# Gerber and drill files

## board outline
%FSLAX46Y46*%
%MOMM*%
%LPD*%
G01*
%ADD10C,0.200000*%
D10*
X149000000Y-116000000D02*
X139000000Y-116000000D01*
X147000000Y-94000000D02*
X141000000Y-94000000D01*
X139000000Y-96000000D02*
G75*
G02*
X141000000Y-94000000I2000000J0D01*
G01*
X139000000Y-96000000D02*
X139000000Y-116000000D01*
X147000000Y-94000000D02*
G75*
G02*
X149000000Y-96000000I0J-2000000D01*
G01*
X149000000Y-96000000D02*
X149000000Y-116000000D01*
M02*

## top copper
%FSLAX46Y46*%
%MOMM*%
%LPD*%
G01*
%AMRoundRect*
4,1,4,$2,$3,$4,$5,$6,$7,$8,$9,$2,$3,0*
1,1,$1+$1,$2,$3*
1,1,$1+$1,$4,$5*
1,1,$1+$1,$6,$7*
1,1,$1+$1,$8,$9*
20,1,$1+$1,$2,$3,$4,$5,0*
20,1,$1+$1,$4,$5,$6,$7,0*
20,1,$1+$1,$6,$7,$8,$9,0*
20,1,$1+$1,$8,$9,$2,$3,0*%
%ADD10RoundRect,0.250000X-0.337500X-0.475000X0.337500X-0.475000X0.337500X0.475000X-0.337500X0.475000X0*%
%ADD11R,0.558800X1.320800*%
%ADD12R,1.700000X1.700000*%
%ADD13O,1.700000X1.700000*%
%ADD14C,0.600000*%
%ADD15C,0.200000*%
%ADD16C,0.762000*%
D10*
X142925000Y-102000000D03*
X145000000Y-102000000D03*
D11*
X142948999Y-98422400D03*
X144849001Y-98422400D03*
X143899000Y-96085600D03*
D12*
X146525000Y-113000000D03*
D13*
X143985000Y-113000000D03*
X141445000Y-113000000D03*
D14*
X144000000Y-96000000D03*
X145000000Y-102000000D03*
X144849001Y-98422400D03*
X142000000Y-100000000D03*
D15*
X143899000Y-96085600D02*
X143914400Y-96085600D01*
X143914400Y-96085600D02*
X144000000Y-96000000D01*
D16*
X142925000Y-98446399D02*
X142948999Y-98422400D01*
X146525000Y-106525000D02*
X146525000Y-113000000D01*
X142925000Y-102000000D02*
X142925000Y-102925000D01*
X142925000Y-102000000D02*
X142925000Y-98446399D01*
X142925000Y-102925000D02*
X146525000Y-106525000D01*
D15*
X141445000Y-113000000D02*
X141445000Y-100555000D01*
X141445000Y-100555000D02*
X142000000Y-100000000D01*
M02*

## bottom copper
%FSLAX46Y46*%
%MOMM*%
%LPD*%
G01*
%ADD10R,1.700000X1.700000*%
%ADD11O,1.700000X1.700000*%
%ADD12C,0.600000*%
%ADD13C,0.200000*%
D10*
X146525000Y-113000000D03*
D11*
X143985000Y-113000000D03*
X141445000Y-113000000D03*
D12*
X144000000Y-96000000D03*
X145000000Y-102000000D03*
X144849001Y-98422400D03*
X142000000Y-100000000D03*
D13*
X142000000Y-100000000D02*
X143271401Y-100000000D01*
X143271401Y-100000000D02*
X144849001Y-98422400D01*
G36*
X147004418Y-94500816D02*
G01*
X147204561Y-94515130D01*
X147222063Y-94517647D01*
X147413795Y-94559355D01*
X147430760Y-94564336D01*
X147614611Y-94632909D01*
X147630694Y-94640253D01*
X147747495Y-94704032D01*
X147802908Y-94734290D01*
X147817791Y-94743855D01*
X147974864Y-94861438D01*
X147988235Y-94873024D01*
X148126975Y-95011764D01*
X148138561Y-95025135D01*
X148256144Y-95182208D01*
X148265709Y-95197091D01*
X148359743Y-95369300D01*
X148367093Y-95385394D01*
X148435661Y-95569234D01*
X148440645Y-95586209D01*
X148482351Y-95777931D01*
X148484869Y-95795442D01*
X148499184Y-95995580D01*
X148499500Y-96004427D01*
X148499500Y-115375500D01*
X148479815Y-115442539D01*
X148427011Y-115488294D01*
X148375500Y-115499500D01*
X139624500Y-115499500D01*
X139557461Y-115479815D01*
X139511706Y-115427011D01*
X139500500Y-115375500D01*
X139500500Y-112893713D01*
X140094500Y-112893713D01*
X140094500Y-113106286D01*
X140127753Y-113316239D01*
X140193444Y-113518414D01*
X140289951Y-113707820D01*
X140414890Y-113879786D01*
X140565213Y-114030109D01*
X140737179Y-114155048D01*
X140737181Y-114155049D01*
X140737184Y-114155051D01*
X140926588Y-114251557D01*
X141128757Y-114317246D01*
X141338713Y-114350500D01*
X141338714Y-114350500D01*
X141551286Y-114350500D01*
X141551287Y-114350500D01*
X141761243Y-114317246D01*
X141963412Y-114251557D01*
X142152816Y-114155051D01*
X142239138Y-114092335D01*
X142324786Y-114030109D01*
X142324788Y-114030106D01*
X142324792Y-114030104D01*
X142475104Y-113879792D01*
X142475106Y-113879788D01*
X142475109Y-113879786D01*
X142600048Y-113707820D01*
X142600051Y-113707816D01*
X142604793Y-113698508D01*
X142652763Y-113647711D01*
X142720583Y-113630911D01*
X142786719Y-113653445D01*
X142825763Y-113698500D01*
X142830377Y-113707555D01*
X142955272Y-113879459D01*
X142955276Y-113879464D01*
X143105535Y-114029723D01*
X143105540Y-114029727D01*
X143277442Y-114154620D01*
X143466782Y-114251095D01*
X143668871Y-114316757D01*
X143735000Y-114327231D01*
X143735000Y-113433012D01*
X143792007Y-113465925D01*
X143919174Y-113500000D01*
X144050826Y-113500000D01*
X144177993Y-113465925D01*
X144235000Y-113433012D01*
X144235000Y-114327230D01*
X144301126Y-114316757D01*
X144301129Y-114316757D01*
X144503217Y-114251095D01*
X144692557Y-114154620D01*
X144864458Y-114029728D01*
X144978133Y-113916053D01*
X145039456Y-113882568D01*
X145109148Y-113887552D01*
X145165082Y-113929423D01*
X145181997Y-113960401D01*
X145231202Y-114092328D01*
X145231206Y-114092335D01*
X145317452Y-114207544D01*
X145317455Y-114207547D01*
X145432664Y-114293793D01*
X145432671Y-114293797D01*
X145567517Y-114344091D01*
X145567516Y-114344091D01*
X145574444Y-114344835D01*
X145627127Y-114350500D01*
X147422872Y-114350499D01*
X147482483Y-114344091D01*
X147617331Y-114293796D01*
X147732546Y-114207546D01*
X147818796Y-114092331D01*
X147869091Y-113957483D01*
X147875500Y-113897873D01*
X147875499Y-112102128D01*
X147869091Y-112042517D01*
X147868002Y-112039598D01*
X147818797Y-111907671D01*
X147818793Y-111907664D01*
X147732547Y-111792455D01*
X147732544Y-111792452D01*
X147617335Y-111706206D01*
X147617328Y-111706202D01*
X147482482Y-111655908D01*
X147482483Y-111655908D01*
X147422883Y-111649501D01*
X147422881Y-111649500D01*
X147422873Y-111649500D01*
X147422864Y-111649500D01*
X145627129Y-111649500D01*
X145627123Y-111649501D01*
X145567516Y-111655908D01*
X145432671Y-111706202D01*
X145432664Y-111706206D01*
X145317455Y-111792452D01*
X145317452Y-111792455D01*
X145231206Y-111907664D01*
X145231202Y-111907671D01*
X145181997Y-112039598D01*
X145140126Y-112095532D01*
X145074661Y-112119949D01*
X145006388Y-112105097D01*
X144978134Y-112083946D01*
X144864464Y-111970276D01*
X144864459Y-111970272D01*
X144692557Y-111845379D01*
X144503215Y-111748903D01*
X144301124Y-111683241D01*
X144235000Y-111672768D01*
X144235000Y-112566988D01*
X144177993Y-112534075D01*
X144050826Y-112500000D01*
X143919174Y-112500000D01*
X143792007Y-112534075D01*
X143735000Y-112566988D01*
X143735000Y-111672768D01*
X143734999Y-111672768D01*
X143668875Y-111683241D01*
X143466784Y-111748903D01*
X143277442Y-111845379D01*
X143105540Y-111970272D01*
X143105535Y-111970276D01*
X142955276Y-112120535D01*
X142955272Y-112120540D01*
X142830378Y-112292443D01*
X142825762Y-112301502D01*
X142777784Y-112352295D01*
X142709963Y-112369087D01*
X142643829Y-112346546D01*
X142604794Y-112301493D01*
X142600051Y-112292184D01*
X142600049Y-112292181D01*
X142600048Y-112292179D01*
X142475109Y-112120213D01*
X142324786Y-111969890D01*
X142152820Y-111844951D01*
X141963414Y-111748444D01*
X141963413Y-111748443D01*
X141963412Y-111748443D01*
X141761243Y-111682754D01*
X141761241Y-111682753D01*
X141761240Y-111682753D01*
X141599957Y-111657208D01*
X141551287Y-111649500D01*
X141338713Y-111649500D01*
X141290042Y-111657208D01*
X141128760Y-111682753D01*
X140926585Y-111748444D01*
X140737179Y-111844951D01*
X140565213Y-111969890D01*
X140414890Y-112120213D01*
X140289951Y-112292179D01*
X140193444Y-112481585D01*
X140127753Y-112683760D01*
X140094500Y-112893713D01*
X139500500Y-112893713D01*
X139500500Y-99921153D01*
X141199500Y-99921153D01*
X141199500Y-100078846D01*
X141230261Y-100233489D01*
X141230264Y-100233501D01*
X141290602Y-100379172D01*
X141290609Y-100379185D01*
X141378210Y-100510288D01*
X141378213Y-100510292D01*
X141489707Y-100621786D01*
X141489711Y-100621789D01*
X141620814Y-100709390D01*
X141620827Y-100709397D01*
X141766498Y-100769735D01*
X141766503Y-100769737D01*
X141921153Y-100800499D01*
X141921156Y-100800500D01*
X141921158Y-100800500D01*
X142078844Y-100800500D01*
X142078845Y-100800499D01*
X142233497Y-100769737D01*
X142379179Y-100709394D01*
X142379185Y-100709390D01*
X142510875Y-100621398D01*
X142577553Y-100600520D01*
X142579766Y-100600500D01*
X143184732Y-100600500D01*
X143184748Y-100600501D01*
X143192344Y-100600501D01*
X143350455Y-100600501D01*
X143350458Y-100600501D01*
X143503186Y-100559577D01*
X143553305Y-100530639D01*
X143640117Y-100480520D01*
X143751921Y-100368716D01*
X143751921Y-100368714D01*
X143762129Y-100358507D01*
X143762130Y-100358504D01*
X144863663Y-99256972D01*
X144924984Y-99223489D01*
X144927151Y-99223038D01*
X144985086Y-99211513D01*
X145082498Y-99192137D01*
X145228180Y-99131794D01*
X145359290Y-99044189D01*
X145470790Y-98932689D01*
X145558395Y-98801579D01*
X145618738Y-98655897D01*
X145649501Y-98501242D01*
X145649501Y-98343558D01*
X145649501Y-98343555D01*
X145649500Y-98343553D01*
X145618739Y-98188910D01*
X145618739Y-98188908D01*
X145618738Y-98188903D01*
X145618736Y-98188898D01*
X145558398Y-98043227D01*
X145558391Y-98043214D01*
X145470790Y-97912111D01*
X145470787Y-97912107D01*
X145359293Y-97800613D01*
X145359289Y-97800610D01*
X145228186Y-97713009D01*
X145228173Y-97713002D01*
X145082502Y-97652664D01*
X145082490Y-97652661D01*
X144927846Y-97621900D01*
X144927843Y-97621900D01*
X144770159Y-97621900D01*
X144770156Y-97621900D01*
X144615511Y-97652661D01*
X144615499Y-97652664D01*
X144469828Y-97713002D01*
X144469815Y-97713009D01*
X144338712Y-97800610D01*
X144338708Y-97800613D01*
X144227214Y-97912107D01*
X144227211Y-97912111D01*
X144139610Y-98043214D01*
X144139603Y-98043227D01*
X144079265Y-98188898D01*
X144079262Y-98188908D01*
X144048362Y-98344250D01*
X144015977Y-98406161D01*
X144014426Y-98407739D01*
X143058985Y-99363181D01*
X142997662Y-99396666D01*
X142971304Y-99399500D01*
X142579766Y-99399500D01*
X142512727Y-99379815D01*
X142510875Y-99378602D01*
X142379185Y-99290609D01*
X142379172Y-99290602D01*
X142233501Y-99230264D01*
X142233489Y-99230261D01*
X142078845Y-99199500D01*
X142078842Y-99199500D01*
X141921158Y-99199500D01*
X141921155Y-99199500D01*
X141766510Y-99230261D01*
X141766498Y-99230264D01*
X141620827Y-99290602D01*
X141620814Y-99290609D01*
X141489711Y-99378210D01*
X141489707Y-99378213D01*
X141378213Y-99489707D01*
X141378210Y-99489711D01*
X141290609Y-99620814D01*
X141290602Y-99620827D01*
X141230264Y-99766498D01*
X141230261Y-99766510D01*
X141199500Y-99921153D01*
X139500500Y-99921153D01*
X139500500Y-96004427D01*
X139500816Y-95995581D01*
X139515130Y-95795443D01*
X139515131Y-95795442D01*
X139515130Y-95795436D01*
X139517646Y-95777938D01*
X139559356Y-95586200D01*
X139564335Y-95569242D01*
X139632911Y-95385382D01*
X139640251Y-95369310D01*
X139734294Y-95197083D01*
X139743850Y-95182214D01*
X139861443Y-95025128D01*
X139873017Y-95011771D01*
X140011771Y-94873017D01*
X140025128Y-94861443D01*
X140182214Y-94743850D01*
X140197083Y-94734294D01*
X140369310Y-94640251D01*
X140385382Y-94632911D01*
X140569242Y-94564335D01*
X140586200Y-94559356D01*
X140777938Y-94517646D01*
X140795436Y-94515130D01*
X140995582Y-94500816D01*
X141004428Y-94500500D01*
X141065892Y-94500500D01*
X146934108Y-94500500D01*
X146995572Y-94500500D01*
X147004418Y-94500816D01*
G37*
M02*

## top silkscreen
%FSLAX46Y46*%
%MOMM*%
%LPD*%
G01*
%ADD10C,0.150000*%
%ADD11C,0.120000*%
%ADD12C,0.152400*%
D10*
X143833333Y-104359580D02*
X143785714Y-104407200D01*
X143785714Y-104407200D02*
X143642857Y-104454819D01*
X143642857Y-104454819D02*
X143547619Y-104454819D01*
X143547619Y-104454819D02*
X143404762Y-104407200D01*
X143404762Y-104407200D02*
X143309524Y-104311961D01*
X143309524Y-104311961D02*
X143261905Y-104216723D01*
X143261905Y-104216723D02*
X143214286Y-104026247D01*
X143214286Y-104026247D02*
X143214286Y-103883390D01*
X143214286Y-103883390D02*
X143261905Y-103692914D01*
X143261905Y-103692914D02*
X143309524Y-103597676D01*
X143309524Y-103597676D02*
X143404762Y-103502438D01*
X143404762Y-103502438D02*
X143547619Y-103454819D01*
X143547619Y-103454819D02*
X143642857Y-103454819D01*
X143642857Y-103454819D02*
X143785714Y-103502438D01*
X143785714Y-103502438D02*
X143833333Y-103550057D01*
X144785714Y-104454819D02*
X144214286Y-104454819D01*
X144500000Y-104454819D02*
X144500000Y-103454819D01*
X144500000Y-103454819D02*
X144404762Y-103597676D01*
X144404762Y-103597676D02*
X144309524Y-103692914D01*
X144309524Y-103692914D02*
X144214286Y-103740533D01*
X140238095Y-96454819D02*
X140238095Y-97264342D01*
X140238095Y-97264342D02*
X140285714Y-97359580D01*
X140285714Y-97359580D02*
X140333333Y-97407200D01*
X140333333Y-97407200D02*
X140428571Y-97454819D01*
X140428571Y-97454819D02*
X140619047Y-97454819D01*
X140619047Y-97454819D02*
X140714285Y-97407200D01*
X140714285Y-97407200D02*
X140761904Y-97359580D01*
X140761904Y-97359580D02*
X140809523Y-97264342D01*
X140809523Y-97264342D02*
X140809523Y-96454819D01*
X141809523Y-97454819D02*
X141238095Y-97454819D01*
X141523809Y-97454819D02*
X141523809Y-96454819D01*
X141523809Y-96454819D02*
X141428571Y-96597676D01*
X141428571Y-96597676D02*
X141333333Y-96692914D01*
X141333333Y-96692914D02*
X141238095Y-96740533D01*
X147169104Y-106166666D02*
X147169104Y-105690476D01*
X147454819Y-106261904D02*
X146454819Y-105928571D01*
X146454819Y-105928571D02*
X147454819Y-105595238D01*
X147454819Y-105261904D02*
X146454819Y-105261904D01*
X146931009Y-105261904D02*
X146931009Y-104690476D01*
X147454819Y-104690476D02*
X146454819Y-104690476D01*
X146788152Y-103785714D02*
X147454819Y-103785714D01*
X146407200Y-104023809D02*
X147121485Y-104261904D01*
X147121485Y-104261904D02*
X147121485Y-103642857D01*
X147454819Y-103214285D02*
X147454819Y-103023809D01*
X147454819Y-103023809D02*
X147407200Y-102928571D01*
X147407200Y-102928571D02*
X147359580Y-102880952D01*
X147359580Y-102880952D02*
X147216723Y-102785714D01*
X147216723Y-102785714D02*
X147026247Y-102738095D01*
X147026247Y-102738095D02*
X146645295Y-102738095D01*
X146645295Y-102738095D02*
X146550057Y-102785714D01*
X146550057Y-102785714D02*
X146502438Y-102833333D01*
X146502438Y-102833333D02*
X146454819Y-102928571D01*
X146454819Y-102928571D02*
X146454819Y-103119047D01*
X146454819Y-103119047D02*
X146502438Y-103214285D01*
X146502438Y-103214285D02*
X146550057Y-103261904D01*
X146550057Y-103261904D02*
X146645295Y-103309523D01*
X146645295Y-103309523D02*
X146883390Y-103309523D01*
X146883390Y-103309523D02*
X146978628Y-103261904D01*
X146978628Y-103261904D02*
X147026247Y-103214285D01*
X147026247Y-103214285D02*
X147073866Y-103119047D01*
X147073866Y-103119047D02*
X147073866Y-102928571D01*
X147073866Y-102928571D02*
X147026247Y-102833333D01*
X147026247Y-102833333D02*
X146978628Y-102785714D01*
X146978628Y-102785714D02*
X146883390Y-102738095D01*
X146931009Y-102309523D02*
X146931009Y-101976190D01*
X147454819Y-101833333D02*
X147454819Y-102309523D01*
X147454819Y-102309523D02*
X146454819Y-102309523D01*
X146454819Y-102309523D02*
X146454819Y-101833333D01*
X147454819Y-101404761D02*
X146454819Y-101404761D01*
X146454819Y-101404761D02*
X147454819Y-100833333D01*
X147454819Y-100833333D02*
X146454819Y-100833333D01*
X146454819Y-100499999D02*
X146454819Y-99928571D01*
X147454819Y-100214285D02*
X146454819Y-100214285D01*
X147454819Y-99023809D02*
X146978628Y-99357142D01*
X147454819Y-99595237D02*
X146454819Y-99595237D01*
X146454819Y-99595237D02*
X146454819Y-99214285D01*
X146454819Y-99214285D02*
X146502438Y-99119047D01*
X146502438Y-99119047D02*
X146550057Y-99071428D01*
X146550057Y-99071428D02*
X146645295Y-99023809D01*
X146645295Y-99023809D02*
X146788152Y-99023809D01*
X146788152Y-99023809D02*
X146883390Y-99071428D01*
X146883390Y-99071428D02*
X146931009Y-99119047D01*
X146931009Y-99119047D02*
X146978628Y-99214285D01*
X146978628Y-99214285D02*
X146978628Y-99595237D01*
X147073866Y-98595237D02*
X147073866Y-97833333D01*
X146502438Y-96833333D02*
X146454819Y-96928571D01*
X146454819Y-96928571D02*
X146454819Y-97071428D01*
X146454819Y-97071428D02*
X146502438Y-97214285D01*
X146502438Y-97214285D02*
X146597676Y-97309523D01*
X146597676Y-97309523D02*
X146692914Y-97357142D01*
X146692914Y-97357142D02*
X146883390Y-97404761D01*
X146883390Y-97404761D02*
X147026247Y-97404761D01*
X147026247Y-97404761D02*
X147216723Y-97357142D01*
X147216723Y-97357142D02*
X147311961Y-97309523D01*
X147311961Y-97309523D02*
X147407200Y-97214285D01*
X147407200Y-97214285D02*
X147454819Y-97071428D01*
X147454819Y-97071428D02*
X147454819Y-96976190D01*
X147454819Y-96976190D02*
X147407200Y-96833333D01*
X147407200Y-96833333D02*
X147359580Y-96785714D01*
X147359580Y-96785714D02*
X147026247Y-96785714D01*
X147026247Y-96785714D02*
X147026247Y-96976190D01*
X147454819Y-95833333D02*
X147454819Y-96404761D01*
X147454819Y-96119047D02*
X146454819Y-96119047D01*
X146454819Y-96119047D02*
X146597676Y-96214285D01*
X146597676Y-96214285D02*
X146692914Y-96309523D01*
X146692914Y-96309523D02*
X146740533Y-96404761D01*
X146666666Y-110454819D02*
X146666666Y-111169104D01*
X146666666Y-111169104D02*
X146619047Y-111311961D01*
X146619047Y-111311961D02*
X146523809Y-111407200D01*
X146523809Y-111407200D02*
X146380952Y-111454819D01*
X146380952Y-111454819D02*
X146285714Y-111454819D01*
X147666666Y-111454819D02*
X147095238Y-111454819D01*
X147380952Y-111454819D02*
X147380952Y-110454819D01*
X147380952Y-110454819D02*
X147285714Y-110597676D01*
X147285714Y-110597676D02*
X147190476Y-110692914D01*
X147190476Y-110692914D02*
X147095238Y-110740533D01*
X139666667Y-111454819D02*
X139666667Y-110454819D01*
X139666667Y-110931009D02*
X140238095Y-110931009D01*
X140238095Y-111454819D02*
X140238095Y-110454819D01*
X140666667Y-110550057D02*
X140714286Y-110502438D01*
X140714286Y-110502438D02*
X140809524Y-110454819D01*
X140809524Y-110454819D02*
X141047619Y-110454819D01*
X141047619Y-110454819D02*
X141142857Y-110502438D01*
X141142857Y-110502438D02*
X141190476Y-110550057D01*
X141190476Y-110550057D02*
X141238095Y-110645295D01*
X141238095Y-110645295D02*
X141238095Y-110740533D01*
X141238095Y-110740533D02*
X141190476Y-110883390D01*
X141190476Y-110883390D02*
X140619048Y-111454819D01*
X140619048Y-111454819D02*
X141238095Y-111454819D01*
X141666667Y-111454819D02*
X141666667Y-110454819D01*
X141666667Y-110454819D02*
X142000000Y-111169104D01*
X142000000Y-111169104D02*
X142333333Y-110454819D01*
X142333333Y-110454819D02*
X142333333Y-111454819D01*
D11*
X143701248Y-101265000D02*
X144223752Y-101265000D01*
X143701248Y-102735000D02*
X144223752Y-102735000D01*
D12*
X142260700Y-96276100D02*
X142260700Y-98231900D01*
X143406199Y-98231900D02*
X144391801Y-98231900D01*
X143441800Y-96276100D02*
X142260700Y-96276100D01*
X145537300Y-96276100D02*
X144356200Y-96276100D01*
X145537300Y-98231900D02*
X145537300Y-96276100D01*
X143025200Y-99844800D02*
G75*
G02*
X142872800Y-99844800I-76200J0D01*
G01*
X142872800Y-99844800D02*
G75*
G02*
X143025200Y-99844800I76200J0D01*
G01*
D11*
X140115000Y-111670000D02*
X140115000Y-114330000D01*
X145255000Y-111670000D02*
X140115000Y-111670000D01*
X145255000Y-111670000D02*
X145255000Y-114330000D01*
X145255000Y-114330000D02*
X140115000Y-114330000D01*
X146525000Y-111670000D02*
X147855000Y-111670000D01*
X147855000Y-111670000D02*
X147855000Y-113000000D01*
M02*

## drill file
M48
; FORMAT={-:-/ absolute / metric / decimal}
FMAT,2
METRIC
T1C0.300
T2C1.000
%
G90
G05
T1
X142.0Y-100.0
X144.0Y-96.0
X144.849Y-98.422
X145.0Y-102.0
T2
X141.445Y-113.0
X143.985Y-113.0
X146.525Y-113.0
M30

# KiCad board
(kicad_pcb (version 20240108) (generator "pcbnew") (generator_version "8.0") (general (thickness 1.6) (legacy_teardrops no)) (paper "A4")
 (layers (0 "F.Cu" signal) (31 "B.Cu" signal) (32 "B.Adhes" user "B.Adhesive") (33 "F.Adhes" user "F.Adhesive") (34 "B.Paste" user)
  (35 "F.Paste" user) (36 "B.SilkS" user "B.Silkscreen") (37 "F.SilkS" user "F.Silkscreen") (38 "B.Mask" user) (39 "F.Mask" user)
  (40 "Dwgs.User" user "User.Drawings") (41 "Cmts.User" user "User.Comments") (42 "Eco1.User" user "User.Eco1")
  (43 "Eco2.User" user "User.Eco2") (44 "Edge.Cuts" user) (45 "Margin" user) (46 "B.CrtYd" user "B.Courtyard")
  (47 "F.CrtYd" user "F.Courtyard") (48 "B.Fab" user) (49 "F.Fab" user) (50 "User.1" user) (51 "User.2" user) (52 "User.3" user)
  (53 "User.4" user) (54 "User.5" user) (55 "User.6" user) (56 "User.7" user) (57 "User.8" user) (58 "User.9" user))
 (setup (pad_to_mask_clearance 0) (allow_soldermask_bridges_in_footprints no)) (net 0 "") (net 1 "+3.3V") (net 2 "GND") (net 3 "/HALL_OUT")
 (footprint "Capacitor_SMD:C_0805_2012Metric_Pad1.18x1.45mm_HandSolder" (layer "F.Cu") (at 143.9625 102)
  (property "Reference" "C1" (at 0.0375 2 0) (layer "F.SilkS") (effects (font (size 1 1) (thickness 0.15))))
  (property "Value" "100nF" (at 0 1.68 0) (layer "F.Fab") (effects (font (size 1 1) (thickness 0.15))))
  (fp_line (start -0.261252 -0.735) (end 0.261252 -0.735) (stroke (width 0.12) (type solid)) (layer "F.SilkS"))
  (fp_line (start -0.261252 0.735) (end 0.261252 0.735) (stroke (width 0.12) (type solid)) (layer "F.SilkS"))
  (pad "1" smd roundrect (at -1.0375 0) (size 1.175 1.45) (layers "F.Cu" "F.Paste" "F.Mask") (roundrect_rratio 0.212766) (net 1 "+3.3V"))
  (pad "2" smd roundrect (at 1.0375 0) (size 1.175 1.45) (layers "F.Cu" "F.Paste" "F.Mask") (roundrect_rratio 0.212766) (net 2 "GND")))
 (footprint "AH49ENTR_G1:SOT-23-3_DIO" (layer "F.Cu") (at 143.899 97.254)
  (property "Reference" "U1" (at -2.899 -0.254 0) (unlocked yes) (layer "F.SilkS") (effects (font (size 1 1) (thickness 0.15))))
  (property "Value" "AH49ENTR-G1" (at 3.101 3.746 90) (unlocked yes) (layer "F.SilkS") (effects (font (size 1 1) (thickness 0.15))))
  (fp_line (start -1.6383 -0.9779) (end -1.6383 0.9779) (stroke (width 0.1524) (type solid)) (layer "F.SilkS"))
  (fp_line (start -0.492801 0.9779) (end 0.492801 0.9779) (stroke (width 0.1524) (type solid)) (layer "F.SilkS"))
  (fp_line (start -0.4572 -0.9779) (end -1.6383 -0.9779) (stroke (width 0.1524) (type solid)) (layer "F.SilkS"))
  (fp_line (start 1.6383 -0.9779) (end 0.4572 -0.9779) (stroke (width 0.1524) (type solid)) (layer "F.SilkS"))
  (fp_line (start 1.6383 0.9779) (end 1.6383 -0.9779) (stroke (width 0.1524) (type solid)) (layer "F.SilkS"))
  (fp_circle (center -0.95 2.5908) (end -0.8738 2.5908) (stroke (width 0.1524) (type solid)) (fill none) (layer "F.SilkS"))
  (pad "1" smd rect (at -0.950001 1.1684) (size 0.5588 1.3208) (layers "F.Cu" "F.Paste" "F.Mask") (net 1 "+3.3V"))
  (pad "2" smd rect (at 0.950001 1.1684) (size 0.5588 1.3208) (layers "F.Cu" "F.Paste" "F.Mask") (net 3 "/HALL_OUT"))
  (pad "3" smd rect (at 0 -1.1684) (size 0.5588 1.3208) (layers "F.Cu" "F.Paste" "F.Mask") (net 2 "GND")))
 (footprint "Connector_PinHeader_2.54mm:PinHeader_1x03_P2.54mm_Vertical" (layer "F.Cu") (at 146.525 113 -90)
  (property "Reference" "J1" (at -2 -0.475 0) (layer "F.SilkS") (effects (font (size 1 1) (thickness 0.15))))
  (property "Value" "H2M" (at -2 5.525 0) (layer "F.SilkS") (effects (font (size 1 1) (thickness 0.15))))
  (fp_line (start -1.33 6.41) (end 1.33 6.41) (stroke (width 0.12) (type solid)) (layer "F.SilkS"))
  (fp_line (start -1.33 1.27) (end -1.33 6.41) (stroke (width 0.12) (type solid)) (layer "F.SilkS"))
  (fp_line (start -1.33 1.27) (end 1.33 1.27) (stroke (width 0.12) (type solid)) (layer "F.SilkS"))
  (fp_line (start 1.33 1.27) (end 1.33 6.41) (stroke (width 0.12) (type solid)) (layer "F.SilkS"))
  (fp_line (start -1.33 0) (end -1.33 -1.33) (stroke (width 0.12) (type solid)) (layer "F.SilkS"))
  (fp_line (start -1.33 -1.33) (end 0 -1.33) (stroke (width 0.12) (type solid)) (layer "F.SilkS"))
  (pad "1" thru_hole rect (at 0 0 270) (size 1.7 1.7) (drill 1) (layers "*.Cu" "*.Mask") (remove_unused_layers no) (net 1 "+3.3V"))
  (pad "2" thru_hole oval (at 0 2.54 270) (size 1.7 1.7) (drill 1) (layers "*.Cu" "*.Mask") (remove_unused_layers no) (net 2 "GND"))
  (pad "3" thru_hole oval (at 0 5.08 270) (size 1.7 1.7) (drill 1) (layers "*.Cu" "*.Mask") (remove_unused_layers no) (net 3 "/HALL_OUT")))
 (gr_line (start 149 116) (end 139 116) (stroke (width 0.2) (type default)) (layer "Edge.Cuts"))
 (gr_line (start 147 94) (end 141 94) (stroke (width 0.2) (type default)) (layer "Edge.Cuts"))
 (gr_arc (start 139 96) (mid 139.585786 94.585786) (end 141 94) (stroke (width 0.2) (type default)) (layer "Edge.Cuts"))
 (gr_line (start 139 96) (end 139 116) (stroke (width 0.2) (type default)) (layer "Edge.Cuts"))
 (gr_arc (start 147 94) (mid 148.414214 94.585786) (end 149 96) (stroke (width 0.2) (type default)) (layer "Edge.Cuts"))
 (gr_line (start 149 96) (end 149 116) (stroke (width 0.2) (type default)) (layer "Edge.Cuts"))
 (segment (start 143.899 96.0856) (end 143.9144 96.0856) (width 0.2) (layer "F.Cu") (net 2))
 (segment (start 143.9144 96.0856) (end 144 96) (width 0.2) (layer "F.Cu") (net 2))
 (via (at 144 96) (size 0.6) (drill 0.3) (layers "F.Cu" "B.Cu") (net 2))
 (via (at 145 102) (size 0.6) (drill 0.3) (layers "F.Cu" "B.Cu") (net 2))
 (segment (start 142.925 98.446399) (end 142.948999 98.4224) (width 0.762) (layer "F.Cu") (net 1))
 (segment (start 146.525 106.525) (end 146.525 113) (width 0.762) (layer "F.Cu") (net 1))
 (segment (start 142.925 102) (end 142.925 102.925) (width 0.762) (layer "F.Cu") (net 1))
 (segment (start 142.925 102) (end 142.925 98.446399) (width 0.762) (layer "F.Cu") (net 1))
 (segment (start 142.925 102.925) (end 146.525 106.525) (width 0.762) (layer "F.Cu") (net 1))
 (segment (start 141.445 113) (end 141.445 100.555) (width 0.2) (layer "F.Cu") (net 3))
 (segment (start 141.445 100.555) (end 142 100) (width 0.2) (layer "F.Cu") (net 3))
 (via (at 144.849001 98.4224) (size 0.6) (drill 0.3) (layers "F.Cu" "B.Cu") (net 3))
 (via (at 142 100) (size 0.6) (drill 0.3) (layers "F.Cu" "B.Cu") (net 3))
 (segment (start 142 100) (end 143.271401 100) (width 0.2) (layer "B.Cu") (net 3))
 (segment (start 143.271401 100) (end 144.849001 98.4224) (width 0.2) (layer "B.Cu") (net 3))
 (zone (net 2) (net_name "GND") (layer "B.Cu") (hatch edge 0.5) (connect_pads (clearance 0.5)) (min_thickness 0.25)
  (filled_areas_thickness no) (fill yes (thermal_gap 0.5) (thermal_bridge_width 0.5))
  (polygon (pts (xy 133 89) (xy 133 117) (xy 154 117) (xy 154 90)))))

